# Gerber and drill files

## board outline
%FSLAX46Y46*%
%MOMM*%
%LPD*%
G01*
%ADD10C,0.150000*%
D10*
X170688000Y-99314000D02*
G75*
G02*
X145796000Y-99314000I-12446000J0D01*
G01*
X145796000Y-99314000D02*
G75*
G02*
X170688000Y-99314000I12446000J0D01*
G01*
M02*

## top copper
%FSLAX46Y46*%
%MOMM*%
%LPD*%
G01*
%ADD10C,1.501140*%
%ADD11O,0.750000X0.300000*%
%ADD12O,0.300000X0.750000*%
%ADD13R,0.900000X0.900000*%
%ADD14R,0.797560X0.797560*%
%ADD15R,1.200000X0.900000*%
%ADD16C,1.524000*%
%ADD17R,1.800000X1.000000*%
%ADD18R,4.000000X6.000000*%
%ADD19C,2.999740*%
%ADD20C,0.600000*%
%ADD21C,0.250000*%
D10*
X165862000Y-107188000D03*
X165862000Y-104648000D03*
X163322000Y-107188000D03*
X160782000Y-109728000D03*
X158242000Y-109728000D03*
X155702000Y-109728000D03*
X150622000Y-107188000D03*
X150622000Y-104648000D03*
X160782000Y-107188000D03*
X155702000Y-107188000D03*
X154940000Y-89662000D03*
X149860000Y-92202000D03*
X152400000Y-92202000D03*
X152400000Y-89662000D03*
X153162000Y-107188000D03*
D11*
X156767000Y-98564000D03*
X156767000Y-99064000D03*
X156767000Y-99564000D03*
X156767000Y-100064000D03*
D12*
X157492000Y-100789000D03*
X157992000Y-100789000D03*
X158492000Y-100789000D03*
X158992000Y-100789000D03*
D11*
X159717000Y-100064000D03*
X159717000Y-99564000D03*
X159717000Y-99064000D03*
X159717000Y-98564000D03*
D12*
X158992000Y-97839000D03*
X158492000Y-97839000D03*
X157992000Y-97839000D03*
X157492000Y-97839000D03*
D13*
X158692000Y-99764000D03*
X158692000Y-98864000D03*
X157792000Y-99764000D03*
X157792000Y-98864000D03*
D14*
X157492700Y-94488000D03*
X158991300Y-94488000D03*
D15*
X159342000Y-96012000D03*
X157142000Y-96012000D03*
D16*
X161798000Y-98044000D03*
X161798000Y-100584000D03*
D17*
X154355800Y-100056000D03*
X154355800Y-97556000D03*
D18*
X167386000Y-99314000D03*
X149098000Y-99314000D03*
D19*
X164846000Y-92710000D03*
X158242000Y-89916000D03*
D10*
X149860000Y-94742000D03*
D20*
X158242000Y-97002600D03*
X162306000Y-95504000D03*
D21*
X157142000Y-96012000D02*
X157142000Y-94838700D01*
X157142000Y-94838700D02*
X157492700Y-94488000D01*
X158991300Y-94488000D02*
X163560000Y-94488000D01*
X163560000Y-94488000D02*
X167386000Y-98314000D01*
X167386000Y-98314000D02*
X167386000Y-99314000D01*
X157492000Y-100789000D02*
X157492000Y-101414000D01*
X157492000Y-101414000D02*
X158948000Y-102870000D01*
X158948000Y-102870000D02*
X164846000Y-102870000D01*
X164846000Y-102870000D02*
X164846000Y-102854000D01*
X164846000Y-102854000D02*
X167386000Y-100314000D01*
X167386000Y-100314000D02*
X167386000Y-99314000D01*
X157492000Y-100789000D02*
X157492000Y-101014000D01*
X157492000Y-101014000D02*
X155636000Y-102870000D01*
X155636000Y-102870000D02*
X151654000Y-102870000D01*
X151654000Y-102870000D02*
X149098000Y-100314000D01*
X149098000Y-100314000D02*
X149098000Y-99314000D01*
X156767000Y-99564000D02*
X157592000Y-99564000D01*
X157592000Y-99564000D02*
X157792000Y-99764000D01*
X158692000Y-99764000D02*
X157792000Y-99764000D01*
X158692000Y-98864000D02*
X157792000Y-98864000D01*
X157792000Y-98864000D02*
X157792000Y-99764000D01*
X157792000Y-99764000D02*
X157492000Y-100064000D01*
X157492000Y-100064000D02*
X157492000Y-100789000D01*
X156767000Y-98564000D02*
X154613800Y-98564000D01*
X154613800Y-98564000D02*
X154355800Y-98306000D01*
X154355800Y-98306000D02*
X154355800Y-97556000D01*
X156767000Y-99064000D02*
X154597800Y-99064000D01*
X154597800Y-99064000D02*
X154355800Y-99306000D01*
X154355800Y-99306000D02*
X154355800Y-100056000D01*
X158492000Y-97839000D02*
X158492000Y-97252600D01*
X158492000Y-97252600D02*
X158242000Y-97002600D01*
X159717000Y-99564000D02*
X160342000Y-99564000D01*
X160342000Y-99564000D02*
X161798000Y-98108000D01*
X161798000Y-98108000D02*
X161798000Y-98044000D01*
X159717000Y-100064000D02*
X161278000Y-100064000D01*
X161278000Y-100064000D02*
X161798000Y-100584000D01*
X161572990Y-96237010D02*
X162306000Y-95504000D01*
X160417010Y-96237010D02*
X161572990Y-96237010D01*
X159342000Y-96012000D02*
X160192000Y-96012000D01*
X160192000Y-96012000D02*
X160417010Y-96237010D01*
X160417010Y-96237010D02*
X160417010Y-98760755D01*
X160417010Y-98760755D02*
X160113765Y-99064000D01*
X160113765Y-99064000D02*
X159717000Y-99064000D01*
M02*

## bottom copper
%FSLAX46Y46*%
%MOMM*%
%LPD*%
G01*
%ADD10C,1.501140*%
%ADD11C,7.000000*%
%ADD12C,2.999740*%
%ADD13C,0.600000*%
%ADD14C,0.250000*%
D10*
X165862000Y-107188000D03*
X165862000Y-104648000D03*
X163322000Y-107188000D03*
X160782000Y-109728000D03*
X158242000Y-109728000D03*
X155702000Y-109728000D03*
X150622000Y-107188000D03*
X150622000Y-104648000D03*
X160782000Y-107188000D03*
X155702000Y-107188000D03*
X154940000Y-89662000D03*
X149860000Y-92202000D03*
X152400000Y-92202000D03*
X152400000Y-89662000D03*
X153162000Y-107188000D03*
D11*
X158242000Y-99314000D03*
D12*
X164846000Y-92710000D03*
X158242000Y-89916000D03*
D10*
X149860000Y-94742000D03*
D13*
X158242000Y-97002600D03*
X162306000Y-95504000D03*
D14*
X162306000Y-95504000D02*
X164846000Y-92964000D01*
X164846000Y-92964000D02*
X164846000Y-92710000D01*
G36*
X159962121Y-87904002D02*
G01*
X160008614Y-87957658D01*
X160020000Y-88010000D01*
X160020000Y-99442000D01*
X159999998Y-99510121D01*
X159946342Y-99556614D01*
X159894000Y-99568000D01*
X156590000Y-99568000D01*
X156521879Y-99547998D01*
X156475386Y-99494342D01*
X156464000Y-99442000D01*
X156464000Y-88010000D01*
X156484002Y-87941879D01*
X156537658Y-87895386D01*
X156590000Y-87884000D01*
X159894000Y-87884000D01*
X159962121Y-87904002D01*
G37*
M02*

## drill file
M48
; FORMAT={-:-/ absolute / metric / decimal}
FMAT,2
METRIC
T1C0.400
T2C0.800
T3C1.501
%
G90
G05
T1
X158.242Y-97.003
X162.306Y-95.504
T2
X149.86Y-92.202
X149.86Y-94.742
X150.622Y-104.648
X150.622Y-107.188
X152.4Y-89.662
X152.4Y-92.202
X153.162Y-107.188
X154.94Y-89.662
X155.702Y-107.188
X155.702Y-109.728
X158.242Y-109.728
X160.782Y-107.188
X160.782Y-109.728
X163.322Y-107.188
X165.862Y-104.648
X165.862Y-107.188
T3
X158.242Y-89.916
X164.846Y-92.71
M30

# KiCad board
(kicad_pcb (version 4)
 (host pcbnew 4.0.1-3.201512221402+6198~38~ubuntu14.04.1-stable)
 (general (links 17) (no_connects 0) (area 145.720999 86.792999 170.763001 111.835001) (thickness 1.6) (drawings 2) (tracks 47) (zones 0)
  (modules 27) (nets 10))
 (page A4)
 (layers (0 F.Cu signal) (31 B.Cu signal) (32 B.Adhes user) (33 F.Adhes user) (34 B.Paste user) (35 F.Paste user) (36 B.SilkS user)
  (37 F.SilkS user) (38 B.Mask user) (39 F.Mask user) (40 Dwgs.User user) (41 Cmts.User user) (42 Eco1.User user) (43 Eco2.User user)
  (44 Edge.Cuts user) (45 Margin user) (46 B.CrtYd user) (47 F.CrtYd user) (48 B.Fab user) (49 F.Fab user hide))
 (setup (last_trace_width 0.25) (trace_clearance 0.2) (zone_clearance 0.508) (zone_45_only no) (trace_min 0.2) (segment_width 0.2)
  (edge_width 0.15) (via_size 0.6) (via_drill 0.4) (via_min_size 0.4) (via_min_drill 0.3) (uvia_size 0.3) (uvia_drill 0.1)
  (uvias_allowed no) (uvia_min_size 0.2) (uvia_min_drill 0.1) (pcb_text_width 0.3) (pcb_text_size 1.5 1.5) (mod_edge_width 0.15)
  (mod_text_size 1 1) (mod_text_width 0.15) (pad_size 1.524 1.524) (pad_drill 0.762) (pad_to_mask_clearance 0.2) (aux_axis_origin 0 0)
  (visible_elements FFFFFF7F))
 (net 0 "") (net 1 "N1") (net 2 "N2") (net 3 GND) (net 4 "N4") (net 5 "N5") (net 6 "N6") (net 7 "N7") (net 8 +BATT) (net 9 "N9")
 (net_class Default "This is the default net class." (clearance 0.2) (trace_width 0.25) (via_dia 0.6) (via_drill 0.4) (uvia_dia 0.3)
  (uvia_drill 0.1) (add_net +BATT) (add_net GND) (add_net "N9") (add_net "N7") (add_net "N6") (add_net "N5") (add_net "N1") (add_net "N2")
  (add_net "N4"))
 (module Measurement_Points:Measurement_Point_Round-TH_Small (layer F.Cu) (at 165.862 107.188)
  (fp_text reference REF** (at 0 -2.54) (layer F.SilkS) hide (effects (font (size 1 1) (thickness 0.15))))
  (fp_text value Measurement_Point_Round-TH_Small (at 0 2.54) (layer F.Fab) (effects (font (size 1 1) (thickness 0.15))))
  (pad 1 thru_hole circle (at 0 0) (size 1.50114 1.50114) (drill 0.8001) (layers *.Cu *.Mask F.SilkS)))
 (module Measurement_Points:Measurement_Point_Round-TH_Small (layer F.Cu) (at 165.862 104.648)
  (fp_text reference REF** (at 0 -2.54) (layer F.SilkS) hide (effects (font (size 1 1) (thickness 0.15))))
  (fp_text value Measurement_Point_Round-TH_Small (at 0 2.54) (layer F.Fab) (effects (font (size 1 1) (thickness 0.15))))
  (pad 1 thru_hole circle (at 0 0) (size 1.50114 1.50114) (drill 0.8001) (layers *.Cu *.Mask F.SilkS)))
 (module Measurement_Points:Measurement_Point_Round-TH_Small (layer F.Cu) (at 163.322 107.188)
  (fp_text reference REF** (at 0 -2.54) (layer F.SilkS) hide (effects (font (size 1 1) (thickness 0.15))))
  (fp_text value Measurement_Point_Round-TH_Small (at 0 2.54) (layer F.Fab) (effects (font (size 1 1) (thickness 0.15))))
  (pad 1 thru_hole circle (at 0 0) (size 1.50114 1.50114) (drill 0.8001) (layers *.Cu *.Mask F.SilkS)))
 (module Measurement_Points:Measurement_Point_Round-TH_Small (layer F.Cu) (at 160.782 109.728)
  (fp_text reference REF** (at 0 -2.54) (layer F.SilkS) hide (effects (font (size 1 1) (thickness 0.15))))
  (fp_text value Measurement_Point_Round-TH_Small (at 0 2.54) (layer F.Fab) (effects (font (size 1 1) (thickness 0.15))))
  (pad 1 thru_hole circle (at 0 0) (size 1.50114 1.50114) (drill 0.8001) (layers *.Cu *.Mask F.SilkS)))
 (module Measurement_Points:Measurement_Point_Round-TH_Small (layer F.Cu) (at 158.242 109.728)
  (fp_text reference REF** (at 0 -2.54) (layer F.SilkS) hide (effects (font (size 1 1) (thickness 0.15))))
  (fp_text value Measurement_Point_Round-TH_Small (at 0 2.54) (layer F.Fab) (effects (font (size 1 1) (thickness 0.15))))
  (pad 1 thru_hole circle (at 0 0) (size 1.50114 1.50114) (drill 0.8001) (layers *.Cu *.Mask F.SilkS)))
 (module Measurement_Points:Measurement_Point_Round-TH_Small (layer F.Cu) (at 155.702 109.728)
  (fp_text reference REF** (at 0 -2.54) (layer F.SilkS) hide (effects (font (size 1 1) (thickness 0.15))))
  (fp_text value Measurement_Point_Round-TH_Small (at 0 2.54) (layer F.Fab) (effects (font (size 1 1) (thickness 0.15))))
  (pad 1 thru_hole circle (at 0 0) (size 1.50114 1.50114) (drill 0.8001) (layers *.Cu *.Mask F.SilkS)))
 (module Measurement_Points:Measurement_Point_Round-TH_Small (layer F.Cu) (at 150.622 107.188)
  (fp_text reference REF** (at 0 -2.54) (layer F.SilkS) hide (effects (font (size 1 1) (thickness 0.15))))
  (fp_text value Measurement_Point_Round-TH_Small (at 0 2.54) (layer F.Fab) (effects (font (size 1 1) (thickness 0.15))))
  (pad 1 thru_hole circle (at 0 0) (size 1.50114 1.50114) (drill 0.8001) (layers *.Cu *.Mask F.SilkS)))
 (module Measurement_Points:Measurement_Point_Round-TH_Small (layer F.Cu) (at 150.622 104.648)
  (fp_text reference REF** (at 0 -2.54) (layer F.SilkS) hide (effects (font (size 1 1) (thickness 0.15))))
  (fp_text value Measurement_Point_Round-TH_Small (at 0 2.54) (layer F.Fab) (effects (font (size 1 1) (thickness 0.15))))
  (pad 1 thru_hole circle (at 0 0) (size 1.50114 1.50114) (drill 0.8001) (layers *.Cu *.Mask F.SilkS)))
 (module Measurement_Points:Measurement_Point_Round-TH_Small (layer F.Cu) (at 160.782 107.188)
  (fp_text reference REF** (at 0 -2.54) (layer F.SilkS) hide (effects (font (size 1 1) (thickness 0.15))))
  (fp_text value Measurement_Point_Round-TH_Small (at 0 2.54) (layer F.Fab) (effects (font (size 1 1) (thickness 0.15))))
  (pad 1 thru_hole circle (at 0 0) (size 1.50114 1.50114) (drill 0.8001) (layers *.Cu *.Mask F.SilkS)))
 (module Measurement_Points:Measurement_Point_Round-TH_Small (layer F.Cu) (at 155.702 107.188)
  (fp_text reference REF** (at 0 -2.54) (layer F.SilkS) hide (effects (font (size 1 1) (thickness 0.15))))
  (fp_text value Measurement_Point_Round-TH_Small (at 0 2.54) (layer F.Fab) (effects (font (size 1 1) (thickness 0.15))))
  (pad 1 thru_hole circle (at 0 0) (size 1.50114 1.50114) (drill 0.8001) (layers *.Cu *.Mask F.SilkS)))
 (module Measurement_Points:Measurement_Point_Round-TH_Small (layer F.Cu) (at 154.94 89.662)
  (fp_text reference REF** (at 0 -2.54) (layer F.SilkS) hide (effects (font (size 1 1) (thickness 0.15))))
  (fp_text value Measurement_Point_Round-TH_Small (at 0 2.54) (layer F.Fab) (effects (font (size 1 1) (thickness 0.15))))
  (pad 1 thru_hole circle (at 0 0) (size 1.50114 1.50114) (drill 0.8001) (layers *.Cu *.Mask F.SilkS)))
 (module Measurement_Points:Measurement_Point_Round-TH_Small (layer F.Cu) (at 149.86 92.202)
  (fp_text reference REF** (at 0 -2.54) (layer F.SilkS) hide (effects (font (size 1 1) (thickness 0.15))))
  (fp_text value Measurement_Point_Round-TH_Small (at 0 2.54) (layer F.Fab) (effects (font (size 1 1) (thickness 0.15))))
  (pad 1 thru_hole circle (at 0 0) (size 1.50114 1.50114) (drill 0.8001) (layers *.Cu *.Mask F.SilkS)))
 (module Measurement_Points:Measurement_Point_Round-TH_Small (layer F.Cu) (at 152.4 92.202)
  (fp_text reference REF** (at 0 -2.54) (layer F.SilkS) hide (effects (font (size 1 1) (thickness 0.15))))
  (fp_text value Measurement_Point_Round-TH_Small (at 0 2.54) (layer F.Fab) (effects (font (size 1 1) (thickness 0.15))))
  (pad 1 thru_hole circle (at 0 0) (size 1.50114 1.50114) (drill 0.8001) (layers *.Cu *.Mask F.SilkS)))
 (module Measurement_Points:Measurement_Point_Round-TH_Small (layer F.Cu) (at 152.4 89.662)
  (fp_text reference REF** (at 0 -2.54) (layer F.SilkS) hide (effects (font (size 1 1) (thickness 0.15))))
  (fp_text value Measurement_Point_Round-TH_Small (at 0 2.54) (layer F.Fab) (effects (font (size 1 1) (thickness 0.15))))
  (pad 1 thru_hole circle (at 0 0) (size 1.50114 1.50114) (drill 0.8001) (layers *.Cu *.Mask F.SilkS)))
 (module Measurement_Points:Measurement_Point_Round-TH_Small (layer F.Cu) (at 153.162 107.188)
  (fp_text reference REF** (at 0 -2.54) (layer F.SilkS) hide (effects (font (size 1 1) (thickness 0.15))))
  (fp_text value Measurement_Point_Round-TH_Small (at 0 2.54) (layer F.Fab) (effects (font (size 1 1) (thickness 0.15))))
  (pad 1 thru_hole circle (at 0 0) (size 1.50114 1.50114) (drill 0.8001) (layers *.Cu *.Mask F.SilkS)))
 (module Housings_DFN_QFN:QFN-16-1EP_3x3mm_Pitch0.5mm (layer F.Cu) (at 158.242 99.314)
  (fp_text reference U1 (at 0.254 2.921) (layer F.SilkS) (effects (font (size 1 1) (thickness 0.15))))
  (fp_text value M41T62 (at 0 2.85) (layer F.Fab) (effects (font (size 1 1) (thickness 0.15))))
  (pad 1 smd oval (at -1.475 -0.75) (size 0.75 0.3) (layers F.Cu F.Paste F.Mask) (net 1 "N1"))
  (pad 2 smd oval (at -1.475 -0.25) (size 0.75 0.3) (layers F.Cu F.Paste F.Mask) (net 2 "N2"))
  (pad 3 smd oval (at -1.475 0.25) (size 0.75 0.3) (layers F.Cu F.Paste F.Mask) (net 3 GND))
  (pad 4 smd oval (at -1.475 0.75) (size 0.75 0.3) (layers F.Cu F.Paste F.Mask) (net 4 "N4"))
  (pad 5 smd oval (at -0.75 1.475 90) (size 0.75 0.3) (layers F.Cu F.Paste F.Mask) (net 3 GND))
  (pad 6 smd oval (at -0.25 1.475 90) (size 0.75 0.3) (layers F.Cu F.Paste F.Mask))
  (pad 7 smd oval (at 0.25 1.475 90) (size 0.75 0.3) (layers F.Cu F.Paste F.Mask))
  (pad 8 smd oval (at 0.75 1.475 90) (size 0.75 0.3) (layers F.Cu F.Paste F.Mask))
  (pad 9 smd oval (at 1.475 0.75) (size 0.75 0.3) (layers F.Cu F.Paste F.Mask) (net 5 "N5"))
  (pad 10 smd oval (at 1.475 0.25) (size 0.75 0.3) (layers F.Cu F.Paste F.Mask) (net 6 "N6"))
  (pad 11 smd oval (at 1.475 -0.25) (size 0.75 0.3) (layers F.Cu F.Paste F.Mask) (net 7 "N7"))
  (pad 12 smd oval (at 1.475 -0.75) (size 0.75 0.3) (layers F.Cu F.Paste F.Mask))
  (pad 13 smd oval (at 0.75 -1.475 90) (size 0.75 0.3) (layers F.Cu F.Paste F.Mask))
  (pad 14 smd oval (at 0.25 -1.475 90) (size 0.75 0.3) (layers F.Cu F.Paste F.Mask) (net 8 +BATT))
  (pad 15 smd oval (at -0.25 -1.475 90) (size 0.75 0.3) (layers F.Cu F.Paste F.Mask))
  (pad 16 smd oval (at -0.75 -1.475 90) (size 0.75 0.3) (layers F.Cu F.Paste F.Mask))
  (pad 17 smd rect (at 0.45 0.45) (size 0.9 0.9) (layers F.Cu F.Paste F.Mask) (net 3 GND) (solder_paste_margin_ratio -0.2))
  (pad 17 smd rect (at 0.45 -0.45) (size 0.9 0.9) (layers F.Cu F.Paste F.Mask) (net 3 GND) (solder_paste_margin_ratio -0.2))
  (pad 17 smd rect (at -0.45 0.45) (size 0.9 0.9) (layers F.Cu F.Paste F.Mask) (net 3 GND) (solder_paste_margin_ratio -0.2))
  (pad 17 smd rect (at -0.45 -0.45) (size 0.9 0.9) (layers F.Cu F.Paste F.Mask) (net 3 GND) (solder_paste_margin_ratio -0.2)))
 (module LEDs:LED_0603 (layer F.Cu) (at 158.242 94.488 180)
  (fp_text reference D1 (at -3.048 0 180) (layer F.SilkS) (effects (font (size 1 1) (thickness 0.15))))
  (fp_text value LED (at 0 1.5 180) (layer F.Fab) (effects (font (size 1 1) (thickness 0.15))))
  (pad 2 smd rect (at 0.7493 0) (size 0.79756 0.79756) (layers F.Cu F.Paste F.Mask) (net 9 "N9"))
  (pad 1 smd rect (at -0.7493 0) (size 0.79756 0.79756) (layers F.Cu F.Paste F.Mask) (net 3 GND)))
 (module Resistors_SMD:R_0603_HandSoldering (layer F.Cu) (at 158.242 96.012 180)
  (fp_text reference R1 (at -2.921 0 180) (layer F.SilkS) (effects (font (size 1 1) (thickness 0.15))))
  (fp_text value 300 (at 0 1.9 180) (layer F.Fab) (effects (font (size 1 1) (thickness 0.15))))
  (pad 1 smd rect (at -1.1 0 180) (size 1.2 0.9) (layers F.Cu F.Paste F.Mask) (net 7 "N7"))
  (pad 2 smd rect (at 1.1 0 180) (size 1.2 0.9) (layers F.Cu F.Paste F.Mask) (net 9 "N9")))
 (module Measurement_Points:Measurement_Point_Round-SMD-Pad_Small (layer F.Cu) (at 161.798 98.044)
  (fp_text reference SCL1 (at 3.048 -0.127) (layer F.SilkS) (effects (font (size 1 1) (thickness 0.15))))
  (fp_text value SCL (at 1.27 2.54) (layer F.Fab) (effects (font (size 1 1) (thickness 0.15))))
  (pad 1 smd circle (at 0 0) (size 1.524 1.524) (layers F.Cu F.Mask) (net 6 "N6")))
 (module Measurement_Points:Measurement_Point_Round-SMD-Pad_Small (layer F.Cu) (at 161.798 100.584)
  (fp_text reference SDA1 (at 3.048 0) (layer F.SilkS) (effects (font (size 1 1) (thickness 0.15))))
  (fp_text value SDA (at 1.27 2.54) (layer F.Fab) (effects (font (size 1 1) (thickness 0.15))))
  (pad 1 smd circle (at 0 0) (size 1.524 1.524) (layers F.Cu F.Mask) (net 5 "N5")))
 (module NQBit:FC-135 (layer F.Cu) (at 154.3558 98.806 270)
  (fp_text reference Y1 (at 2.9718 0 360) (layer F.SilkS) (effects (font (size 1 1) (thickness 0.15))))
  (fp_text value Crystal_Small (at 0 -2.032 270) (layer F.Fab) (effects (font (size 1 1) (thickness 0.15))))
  (pad 1 smd rect (at 1.25 0 270) (size 1 1.8) (layers F.Cu F.Paste F.Mask) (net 2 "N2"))
  (pad 2 smd rect (at -1.25 0 270) (size 1 1.8) (layers F.Cu F.Paste F.Mask) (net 1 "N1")))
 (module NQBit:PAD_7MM (layer B.Cu) (at 158.242 99.314)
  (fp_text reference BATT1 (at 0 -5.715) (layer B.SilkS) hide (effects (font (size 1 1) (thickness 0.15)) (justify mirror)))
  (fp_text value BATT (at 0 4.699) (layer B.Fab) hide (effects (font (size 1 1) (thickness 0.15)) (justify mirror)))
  (pad 1 smd circle (at 0 0) (size 7 7) (layers B.Cu B.Paste B.Mask) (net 8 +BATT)))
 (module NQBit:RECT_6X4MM (layer F.Cu) (at 167.386 99.314)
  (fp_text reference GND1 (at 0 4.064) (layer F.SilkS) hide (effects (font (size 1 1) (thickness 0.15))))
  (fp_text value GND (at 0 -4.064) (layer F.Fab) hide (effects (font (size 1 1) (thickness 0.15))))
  (pad 1 smd rect (at 0 0) (size 4 6) (layers F.Cu F.Paste F.Mask) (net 3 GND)))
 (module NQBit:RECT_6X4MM (layer F.Cu) (at 149.098 99.314)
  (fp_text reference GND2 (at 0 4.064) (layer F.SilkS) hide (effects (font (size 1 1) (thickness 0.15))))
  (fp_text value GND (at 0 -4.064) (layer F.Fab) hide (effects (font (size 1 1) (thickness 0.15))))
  (pad 1 smd rect (at 0 0) (size 4 6) (layers F.Cu F.Paste F.Mask) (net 3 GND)))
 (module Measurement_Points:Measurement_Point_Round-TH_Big (layer F.Cu) (at 164.846 92.71)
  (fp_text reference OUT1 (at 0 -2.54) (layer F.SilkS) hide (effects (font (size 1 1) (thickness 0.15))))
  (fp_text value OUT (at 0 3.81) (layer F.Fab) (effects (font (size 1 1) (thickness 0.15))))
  (pad 1 thru_hole circle (at 0 0) (size 2.99974 2.99974) (drill 1.50114) (layers *.Cu *.Mask F.SilkS) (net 7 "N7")))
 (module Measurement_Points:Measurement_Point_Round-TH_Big (layer F.Cu) (at 158.242 89.916)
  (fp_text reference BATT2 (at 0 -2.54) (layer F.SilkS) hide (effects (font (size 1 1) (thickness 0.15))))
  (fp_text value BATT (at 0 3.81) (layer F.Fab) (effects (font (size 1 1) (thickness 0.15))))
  (pad 1 thru_hole circle (at 0 0) (size 2.99974 2.99974) (drill 1.50114) (layers *.Cu *.Mask F.SilkS) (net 8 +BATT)))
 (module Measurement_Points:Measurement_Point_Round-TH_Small (layer F.Cu) (at 149.86 94.742)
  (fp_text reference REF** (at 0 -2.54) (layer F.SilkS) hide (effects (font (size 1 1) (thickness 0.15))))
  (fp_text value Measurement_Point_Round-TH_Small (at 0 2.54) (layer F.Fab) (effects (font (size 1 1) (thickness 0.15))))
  (pad 1 thru_hole circle (at 0 0) (size 1.50114 1.50114) (drill 0.8001) (layers *.Cu *.Mask F.SilkS)))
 (gr_circle (center 158.242 99.314) (end 158.242 86.868) (layer Edge.Cuts) (width 0.15))
 (segment (start 157.142 96.012) (end 157.142 94.8387) (width 0.25) (layer F.Cu) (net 9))
 (segment (start 157.142 94.8387) (end 157.4927 94.488) (width 0.25) (layer F.Cu) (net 9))
 (segment (start 158.9913 94.488) (end 163.56 94.488) (width 0.25) (layer F.Cu) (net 3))
 (segment (start 163.56 94.488) (end 167.386 98.314) (width 0.25) (layer F.Cu) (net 3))
 (segment (start 167.386 98.314) (end 167.386 99.314) (width 0.25) (layer F.Cu) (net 3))
 (segment (start 157.492 100.789) (end 157.492 101.414) (width 0.25) (layer F.Cu) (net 3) (status 10))
 (segment (start 157.492 101.414) (end 158.948 102.87) (width 0.25) (layer F.Cu) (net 3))
 (segment (start 158.948 102.87) (end 164.846 102.87) (width 0.25) (layer F.Cu) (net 3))
 (segment (start 164.846 102.87) (end 164.846 102.854) (width 0.25) (layer F.Cu) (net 3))
 (segment (start 164.846 102.854) (end 167.386 100.314) (width 0.25) (layer F.Cu) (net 3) (status 20))
 (segment (start 167.386 100.314) (end 167.386 99.314) (width 0.25) (layer F.Cu) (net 3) (status 30))
 (segment (start 157.492 100.789) (end 157.492 101.014) (width 0.25) (layer F.Cu) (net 3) (status 30))
 (segment (start 157.492 101.014) (end 155.636 102.87) (width 0.25) (layer F.Cu) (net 3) (status 10))
 (segment (start 155.636 102.87) (end 151.654 102.87) (width 0.25) (layer F.Cu) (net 3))
 (segment (start 151.654 102.87) (end 149.098 100.314) (width 0.25) (layer F.Cu) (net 3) (status 20))
 (segment (start 149.098 100.314) (end 149.098 99.314) (width 0.25) (layer F.Cu) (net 3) (status 30))
 (segment (start 156.767 99.564) (end 157.592 99.564) (width 0.25) (layer F.Cu) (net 3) (status 30))
 (segment (start 157.592 99.564) (end 157.792 99.764) (width 0.25) (layer F.Cu) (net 3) (status 30))
 (segment (start 158.692 99.764) (end 157.792 99.764) (width 0.25) (layer F.Cu) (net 3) (status 30))
 (segment (start 158.692 98.864) (end 157.792 98.864) (width 0.25) (layer F.Cu) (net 3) (status 30))
 (segment (start 157.792 98.864) (end 157.792 99.764) (width 0.25) (layer F.Cu) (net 3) (status 30))
 (segment (start 157.792 99.764) (end 157.492 100.064) (width 0.25) (layer F.Cu) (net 3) (status 30))
 (segment (start 157.492 100.064) (end 157.492 100.789) (width 0.25) (layer F.Cu) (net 3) (status 30))
 (segment (start 156.767 98.564) (end 154.6138 98.564) (width 0.25) (layer F.Cu) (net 1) (status 10))
 (segment (start 154.6138 98.564) (end 154.3558 98.306) (width 0.25) (layer F.Cu) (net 1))
 (segment (start 154.3558 98.306) (end 154.3558 97.556) (width 0.25) (layer F.Cu) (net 1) (status 20))
 (segment (start 156.767 99.064) (end 154.5978 99.064) (width 0.25) (layer F.Cu) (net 2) (status 10))
 (segment (start 154.5978 99.064) (end 154.3558 99.306) (width 0.25) (layer F.Cu) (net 2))
 (segment (start 154.3558 99.306) (end 154.3558 100.056) (width 0.25) (layer F.Cu) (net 2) (status 20))
 (segment (start 158.492 97.839) (end 158.492 97.2526) (width 0.25) (layer F.Cu) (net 8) (status 10))
 (segment (start 158.492 97.2526) (end 158.242 97.0026) (width 0.25) (layer F.Cu) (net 8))
 (via (at 158.242 97.0026) (size 0.6) (drill 0.4) (layers F.Cu B.Cu) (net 8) (status 30))
 (segment (start 159.717 99.564) (end 160.342 99.564) (width 0.25) (layer F.Cu) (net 6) (status 10))
 (segment (start 160.342 99.564) (end 161.798 98.108) (width 0.25) (layer F.Cu) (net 6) (status 20))
 (segment (start 161.798 98.108) (end 161.798 98.044) (width 0.25) (layer F.Cu) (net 6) (status 30))
 (segment (start 159.717 100.064) (end 161.278 100.064) (width 0.25) (layer F.Cu) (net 5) (status 30))
 (segment (start 161.278 100.064) (end 161.798 100.584) (width 0.25) (layer F.Cu) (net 5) (status 30))
 (segment (start 162.306 95.504) (end 164.846 92.964) (width 0.25) (layer B.Cu) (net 7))
 (segment (start 164.846 92.964) (end 164.846 92.71) (width 0.25) (layer B.Cu) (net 7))
 (segment (start 161.57299 96.23701) (end 162.306 95.504) (width 0.25) (layer F.Cu) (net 7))
 (via (at 162.306 95.504) (size 0.6) (drill 0.4) (layers F.Cu B.Cu) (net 7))
 (segment (start 160.41701 96.23701) (end 161.57299 96.23701) (width 0.25) (layer F.Cu) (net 7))
 (segment (start 159.342 96.012) (end 160.192 96.012) (width 0.25) (layer F.Cu) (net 7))
 (segment (start 160.192 96.012) (end 160.41701 96.23701) (width 0.25) (layer F.Cu) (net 7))
 (segment (start 160.41701 96.23701) (end 160.41701 98.760755) (width 0.25) (layer F.Cu) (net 7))
 (segment (start 160.41701 98.760755) (end 160.113765 99.064) (width 0.25) (layer F.Cu) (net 7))
 (segment (start 160.113765 99.064) (end 159.717 99.064) (width 0.25) (layer F.Cu) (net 7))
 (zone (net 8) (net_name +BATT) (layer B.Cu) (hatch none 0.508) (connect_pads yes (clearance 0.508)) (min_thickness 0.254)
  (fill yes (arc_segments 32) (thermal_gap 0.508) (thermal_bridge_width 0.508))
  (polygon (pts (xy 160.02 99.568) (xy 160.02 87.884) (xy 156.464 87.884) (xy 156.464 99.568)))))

